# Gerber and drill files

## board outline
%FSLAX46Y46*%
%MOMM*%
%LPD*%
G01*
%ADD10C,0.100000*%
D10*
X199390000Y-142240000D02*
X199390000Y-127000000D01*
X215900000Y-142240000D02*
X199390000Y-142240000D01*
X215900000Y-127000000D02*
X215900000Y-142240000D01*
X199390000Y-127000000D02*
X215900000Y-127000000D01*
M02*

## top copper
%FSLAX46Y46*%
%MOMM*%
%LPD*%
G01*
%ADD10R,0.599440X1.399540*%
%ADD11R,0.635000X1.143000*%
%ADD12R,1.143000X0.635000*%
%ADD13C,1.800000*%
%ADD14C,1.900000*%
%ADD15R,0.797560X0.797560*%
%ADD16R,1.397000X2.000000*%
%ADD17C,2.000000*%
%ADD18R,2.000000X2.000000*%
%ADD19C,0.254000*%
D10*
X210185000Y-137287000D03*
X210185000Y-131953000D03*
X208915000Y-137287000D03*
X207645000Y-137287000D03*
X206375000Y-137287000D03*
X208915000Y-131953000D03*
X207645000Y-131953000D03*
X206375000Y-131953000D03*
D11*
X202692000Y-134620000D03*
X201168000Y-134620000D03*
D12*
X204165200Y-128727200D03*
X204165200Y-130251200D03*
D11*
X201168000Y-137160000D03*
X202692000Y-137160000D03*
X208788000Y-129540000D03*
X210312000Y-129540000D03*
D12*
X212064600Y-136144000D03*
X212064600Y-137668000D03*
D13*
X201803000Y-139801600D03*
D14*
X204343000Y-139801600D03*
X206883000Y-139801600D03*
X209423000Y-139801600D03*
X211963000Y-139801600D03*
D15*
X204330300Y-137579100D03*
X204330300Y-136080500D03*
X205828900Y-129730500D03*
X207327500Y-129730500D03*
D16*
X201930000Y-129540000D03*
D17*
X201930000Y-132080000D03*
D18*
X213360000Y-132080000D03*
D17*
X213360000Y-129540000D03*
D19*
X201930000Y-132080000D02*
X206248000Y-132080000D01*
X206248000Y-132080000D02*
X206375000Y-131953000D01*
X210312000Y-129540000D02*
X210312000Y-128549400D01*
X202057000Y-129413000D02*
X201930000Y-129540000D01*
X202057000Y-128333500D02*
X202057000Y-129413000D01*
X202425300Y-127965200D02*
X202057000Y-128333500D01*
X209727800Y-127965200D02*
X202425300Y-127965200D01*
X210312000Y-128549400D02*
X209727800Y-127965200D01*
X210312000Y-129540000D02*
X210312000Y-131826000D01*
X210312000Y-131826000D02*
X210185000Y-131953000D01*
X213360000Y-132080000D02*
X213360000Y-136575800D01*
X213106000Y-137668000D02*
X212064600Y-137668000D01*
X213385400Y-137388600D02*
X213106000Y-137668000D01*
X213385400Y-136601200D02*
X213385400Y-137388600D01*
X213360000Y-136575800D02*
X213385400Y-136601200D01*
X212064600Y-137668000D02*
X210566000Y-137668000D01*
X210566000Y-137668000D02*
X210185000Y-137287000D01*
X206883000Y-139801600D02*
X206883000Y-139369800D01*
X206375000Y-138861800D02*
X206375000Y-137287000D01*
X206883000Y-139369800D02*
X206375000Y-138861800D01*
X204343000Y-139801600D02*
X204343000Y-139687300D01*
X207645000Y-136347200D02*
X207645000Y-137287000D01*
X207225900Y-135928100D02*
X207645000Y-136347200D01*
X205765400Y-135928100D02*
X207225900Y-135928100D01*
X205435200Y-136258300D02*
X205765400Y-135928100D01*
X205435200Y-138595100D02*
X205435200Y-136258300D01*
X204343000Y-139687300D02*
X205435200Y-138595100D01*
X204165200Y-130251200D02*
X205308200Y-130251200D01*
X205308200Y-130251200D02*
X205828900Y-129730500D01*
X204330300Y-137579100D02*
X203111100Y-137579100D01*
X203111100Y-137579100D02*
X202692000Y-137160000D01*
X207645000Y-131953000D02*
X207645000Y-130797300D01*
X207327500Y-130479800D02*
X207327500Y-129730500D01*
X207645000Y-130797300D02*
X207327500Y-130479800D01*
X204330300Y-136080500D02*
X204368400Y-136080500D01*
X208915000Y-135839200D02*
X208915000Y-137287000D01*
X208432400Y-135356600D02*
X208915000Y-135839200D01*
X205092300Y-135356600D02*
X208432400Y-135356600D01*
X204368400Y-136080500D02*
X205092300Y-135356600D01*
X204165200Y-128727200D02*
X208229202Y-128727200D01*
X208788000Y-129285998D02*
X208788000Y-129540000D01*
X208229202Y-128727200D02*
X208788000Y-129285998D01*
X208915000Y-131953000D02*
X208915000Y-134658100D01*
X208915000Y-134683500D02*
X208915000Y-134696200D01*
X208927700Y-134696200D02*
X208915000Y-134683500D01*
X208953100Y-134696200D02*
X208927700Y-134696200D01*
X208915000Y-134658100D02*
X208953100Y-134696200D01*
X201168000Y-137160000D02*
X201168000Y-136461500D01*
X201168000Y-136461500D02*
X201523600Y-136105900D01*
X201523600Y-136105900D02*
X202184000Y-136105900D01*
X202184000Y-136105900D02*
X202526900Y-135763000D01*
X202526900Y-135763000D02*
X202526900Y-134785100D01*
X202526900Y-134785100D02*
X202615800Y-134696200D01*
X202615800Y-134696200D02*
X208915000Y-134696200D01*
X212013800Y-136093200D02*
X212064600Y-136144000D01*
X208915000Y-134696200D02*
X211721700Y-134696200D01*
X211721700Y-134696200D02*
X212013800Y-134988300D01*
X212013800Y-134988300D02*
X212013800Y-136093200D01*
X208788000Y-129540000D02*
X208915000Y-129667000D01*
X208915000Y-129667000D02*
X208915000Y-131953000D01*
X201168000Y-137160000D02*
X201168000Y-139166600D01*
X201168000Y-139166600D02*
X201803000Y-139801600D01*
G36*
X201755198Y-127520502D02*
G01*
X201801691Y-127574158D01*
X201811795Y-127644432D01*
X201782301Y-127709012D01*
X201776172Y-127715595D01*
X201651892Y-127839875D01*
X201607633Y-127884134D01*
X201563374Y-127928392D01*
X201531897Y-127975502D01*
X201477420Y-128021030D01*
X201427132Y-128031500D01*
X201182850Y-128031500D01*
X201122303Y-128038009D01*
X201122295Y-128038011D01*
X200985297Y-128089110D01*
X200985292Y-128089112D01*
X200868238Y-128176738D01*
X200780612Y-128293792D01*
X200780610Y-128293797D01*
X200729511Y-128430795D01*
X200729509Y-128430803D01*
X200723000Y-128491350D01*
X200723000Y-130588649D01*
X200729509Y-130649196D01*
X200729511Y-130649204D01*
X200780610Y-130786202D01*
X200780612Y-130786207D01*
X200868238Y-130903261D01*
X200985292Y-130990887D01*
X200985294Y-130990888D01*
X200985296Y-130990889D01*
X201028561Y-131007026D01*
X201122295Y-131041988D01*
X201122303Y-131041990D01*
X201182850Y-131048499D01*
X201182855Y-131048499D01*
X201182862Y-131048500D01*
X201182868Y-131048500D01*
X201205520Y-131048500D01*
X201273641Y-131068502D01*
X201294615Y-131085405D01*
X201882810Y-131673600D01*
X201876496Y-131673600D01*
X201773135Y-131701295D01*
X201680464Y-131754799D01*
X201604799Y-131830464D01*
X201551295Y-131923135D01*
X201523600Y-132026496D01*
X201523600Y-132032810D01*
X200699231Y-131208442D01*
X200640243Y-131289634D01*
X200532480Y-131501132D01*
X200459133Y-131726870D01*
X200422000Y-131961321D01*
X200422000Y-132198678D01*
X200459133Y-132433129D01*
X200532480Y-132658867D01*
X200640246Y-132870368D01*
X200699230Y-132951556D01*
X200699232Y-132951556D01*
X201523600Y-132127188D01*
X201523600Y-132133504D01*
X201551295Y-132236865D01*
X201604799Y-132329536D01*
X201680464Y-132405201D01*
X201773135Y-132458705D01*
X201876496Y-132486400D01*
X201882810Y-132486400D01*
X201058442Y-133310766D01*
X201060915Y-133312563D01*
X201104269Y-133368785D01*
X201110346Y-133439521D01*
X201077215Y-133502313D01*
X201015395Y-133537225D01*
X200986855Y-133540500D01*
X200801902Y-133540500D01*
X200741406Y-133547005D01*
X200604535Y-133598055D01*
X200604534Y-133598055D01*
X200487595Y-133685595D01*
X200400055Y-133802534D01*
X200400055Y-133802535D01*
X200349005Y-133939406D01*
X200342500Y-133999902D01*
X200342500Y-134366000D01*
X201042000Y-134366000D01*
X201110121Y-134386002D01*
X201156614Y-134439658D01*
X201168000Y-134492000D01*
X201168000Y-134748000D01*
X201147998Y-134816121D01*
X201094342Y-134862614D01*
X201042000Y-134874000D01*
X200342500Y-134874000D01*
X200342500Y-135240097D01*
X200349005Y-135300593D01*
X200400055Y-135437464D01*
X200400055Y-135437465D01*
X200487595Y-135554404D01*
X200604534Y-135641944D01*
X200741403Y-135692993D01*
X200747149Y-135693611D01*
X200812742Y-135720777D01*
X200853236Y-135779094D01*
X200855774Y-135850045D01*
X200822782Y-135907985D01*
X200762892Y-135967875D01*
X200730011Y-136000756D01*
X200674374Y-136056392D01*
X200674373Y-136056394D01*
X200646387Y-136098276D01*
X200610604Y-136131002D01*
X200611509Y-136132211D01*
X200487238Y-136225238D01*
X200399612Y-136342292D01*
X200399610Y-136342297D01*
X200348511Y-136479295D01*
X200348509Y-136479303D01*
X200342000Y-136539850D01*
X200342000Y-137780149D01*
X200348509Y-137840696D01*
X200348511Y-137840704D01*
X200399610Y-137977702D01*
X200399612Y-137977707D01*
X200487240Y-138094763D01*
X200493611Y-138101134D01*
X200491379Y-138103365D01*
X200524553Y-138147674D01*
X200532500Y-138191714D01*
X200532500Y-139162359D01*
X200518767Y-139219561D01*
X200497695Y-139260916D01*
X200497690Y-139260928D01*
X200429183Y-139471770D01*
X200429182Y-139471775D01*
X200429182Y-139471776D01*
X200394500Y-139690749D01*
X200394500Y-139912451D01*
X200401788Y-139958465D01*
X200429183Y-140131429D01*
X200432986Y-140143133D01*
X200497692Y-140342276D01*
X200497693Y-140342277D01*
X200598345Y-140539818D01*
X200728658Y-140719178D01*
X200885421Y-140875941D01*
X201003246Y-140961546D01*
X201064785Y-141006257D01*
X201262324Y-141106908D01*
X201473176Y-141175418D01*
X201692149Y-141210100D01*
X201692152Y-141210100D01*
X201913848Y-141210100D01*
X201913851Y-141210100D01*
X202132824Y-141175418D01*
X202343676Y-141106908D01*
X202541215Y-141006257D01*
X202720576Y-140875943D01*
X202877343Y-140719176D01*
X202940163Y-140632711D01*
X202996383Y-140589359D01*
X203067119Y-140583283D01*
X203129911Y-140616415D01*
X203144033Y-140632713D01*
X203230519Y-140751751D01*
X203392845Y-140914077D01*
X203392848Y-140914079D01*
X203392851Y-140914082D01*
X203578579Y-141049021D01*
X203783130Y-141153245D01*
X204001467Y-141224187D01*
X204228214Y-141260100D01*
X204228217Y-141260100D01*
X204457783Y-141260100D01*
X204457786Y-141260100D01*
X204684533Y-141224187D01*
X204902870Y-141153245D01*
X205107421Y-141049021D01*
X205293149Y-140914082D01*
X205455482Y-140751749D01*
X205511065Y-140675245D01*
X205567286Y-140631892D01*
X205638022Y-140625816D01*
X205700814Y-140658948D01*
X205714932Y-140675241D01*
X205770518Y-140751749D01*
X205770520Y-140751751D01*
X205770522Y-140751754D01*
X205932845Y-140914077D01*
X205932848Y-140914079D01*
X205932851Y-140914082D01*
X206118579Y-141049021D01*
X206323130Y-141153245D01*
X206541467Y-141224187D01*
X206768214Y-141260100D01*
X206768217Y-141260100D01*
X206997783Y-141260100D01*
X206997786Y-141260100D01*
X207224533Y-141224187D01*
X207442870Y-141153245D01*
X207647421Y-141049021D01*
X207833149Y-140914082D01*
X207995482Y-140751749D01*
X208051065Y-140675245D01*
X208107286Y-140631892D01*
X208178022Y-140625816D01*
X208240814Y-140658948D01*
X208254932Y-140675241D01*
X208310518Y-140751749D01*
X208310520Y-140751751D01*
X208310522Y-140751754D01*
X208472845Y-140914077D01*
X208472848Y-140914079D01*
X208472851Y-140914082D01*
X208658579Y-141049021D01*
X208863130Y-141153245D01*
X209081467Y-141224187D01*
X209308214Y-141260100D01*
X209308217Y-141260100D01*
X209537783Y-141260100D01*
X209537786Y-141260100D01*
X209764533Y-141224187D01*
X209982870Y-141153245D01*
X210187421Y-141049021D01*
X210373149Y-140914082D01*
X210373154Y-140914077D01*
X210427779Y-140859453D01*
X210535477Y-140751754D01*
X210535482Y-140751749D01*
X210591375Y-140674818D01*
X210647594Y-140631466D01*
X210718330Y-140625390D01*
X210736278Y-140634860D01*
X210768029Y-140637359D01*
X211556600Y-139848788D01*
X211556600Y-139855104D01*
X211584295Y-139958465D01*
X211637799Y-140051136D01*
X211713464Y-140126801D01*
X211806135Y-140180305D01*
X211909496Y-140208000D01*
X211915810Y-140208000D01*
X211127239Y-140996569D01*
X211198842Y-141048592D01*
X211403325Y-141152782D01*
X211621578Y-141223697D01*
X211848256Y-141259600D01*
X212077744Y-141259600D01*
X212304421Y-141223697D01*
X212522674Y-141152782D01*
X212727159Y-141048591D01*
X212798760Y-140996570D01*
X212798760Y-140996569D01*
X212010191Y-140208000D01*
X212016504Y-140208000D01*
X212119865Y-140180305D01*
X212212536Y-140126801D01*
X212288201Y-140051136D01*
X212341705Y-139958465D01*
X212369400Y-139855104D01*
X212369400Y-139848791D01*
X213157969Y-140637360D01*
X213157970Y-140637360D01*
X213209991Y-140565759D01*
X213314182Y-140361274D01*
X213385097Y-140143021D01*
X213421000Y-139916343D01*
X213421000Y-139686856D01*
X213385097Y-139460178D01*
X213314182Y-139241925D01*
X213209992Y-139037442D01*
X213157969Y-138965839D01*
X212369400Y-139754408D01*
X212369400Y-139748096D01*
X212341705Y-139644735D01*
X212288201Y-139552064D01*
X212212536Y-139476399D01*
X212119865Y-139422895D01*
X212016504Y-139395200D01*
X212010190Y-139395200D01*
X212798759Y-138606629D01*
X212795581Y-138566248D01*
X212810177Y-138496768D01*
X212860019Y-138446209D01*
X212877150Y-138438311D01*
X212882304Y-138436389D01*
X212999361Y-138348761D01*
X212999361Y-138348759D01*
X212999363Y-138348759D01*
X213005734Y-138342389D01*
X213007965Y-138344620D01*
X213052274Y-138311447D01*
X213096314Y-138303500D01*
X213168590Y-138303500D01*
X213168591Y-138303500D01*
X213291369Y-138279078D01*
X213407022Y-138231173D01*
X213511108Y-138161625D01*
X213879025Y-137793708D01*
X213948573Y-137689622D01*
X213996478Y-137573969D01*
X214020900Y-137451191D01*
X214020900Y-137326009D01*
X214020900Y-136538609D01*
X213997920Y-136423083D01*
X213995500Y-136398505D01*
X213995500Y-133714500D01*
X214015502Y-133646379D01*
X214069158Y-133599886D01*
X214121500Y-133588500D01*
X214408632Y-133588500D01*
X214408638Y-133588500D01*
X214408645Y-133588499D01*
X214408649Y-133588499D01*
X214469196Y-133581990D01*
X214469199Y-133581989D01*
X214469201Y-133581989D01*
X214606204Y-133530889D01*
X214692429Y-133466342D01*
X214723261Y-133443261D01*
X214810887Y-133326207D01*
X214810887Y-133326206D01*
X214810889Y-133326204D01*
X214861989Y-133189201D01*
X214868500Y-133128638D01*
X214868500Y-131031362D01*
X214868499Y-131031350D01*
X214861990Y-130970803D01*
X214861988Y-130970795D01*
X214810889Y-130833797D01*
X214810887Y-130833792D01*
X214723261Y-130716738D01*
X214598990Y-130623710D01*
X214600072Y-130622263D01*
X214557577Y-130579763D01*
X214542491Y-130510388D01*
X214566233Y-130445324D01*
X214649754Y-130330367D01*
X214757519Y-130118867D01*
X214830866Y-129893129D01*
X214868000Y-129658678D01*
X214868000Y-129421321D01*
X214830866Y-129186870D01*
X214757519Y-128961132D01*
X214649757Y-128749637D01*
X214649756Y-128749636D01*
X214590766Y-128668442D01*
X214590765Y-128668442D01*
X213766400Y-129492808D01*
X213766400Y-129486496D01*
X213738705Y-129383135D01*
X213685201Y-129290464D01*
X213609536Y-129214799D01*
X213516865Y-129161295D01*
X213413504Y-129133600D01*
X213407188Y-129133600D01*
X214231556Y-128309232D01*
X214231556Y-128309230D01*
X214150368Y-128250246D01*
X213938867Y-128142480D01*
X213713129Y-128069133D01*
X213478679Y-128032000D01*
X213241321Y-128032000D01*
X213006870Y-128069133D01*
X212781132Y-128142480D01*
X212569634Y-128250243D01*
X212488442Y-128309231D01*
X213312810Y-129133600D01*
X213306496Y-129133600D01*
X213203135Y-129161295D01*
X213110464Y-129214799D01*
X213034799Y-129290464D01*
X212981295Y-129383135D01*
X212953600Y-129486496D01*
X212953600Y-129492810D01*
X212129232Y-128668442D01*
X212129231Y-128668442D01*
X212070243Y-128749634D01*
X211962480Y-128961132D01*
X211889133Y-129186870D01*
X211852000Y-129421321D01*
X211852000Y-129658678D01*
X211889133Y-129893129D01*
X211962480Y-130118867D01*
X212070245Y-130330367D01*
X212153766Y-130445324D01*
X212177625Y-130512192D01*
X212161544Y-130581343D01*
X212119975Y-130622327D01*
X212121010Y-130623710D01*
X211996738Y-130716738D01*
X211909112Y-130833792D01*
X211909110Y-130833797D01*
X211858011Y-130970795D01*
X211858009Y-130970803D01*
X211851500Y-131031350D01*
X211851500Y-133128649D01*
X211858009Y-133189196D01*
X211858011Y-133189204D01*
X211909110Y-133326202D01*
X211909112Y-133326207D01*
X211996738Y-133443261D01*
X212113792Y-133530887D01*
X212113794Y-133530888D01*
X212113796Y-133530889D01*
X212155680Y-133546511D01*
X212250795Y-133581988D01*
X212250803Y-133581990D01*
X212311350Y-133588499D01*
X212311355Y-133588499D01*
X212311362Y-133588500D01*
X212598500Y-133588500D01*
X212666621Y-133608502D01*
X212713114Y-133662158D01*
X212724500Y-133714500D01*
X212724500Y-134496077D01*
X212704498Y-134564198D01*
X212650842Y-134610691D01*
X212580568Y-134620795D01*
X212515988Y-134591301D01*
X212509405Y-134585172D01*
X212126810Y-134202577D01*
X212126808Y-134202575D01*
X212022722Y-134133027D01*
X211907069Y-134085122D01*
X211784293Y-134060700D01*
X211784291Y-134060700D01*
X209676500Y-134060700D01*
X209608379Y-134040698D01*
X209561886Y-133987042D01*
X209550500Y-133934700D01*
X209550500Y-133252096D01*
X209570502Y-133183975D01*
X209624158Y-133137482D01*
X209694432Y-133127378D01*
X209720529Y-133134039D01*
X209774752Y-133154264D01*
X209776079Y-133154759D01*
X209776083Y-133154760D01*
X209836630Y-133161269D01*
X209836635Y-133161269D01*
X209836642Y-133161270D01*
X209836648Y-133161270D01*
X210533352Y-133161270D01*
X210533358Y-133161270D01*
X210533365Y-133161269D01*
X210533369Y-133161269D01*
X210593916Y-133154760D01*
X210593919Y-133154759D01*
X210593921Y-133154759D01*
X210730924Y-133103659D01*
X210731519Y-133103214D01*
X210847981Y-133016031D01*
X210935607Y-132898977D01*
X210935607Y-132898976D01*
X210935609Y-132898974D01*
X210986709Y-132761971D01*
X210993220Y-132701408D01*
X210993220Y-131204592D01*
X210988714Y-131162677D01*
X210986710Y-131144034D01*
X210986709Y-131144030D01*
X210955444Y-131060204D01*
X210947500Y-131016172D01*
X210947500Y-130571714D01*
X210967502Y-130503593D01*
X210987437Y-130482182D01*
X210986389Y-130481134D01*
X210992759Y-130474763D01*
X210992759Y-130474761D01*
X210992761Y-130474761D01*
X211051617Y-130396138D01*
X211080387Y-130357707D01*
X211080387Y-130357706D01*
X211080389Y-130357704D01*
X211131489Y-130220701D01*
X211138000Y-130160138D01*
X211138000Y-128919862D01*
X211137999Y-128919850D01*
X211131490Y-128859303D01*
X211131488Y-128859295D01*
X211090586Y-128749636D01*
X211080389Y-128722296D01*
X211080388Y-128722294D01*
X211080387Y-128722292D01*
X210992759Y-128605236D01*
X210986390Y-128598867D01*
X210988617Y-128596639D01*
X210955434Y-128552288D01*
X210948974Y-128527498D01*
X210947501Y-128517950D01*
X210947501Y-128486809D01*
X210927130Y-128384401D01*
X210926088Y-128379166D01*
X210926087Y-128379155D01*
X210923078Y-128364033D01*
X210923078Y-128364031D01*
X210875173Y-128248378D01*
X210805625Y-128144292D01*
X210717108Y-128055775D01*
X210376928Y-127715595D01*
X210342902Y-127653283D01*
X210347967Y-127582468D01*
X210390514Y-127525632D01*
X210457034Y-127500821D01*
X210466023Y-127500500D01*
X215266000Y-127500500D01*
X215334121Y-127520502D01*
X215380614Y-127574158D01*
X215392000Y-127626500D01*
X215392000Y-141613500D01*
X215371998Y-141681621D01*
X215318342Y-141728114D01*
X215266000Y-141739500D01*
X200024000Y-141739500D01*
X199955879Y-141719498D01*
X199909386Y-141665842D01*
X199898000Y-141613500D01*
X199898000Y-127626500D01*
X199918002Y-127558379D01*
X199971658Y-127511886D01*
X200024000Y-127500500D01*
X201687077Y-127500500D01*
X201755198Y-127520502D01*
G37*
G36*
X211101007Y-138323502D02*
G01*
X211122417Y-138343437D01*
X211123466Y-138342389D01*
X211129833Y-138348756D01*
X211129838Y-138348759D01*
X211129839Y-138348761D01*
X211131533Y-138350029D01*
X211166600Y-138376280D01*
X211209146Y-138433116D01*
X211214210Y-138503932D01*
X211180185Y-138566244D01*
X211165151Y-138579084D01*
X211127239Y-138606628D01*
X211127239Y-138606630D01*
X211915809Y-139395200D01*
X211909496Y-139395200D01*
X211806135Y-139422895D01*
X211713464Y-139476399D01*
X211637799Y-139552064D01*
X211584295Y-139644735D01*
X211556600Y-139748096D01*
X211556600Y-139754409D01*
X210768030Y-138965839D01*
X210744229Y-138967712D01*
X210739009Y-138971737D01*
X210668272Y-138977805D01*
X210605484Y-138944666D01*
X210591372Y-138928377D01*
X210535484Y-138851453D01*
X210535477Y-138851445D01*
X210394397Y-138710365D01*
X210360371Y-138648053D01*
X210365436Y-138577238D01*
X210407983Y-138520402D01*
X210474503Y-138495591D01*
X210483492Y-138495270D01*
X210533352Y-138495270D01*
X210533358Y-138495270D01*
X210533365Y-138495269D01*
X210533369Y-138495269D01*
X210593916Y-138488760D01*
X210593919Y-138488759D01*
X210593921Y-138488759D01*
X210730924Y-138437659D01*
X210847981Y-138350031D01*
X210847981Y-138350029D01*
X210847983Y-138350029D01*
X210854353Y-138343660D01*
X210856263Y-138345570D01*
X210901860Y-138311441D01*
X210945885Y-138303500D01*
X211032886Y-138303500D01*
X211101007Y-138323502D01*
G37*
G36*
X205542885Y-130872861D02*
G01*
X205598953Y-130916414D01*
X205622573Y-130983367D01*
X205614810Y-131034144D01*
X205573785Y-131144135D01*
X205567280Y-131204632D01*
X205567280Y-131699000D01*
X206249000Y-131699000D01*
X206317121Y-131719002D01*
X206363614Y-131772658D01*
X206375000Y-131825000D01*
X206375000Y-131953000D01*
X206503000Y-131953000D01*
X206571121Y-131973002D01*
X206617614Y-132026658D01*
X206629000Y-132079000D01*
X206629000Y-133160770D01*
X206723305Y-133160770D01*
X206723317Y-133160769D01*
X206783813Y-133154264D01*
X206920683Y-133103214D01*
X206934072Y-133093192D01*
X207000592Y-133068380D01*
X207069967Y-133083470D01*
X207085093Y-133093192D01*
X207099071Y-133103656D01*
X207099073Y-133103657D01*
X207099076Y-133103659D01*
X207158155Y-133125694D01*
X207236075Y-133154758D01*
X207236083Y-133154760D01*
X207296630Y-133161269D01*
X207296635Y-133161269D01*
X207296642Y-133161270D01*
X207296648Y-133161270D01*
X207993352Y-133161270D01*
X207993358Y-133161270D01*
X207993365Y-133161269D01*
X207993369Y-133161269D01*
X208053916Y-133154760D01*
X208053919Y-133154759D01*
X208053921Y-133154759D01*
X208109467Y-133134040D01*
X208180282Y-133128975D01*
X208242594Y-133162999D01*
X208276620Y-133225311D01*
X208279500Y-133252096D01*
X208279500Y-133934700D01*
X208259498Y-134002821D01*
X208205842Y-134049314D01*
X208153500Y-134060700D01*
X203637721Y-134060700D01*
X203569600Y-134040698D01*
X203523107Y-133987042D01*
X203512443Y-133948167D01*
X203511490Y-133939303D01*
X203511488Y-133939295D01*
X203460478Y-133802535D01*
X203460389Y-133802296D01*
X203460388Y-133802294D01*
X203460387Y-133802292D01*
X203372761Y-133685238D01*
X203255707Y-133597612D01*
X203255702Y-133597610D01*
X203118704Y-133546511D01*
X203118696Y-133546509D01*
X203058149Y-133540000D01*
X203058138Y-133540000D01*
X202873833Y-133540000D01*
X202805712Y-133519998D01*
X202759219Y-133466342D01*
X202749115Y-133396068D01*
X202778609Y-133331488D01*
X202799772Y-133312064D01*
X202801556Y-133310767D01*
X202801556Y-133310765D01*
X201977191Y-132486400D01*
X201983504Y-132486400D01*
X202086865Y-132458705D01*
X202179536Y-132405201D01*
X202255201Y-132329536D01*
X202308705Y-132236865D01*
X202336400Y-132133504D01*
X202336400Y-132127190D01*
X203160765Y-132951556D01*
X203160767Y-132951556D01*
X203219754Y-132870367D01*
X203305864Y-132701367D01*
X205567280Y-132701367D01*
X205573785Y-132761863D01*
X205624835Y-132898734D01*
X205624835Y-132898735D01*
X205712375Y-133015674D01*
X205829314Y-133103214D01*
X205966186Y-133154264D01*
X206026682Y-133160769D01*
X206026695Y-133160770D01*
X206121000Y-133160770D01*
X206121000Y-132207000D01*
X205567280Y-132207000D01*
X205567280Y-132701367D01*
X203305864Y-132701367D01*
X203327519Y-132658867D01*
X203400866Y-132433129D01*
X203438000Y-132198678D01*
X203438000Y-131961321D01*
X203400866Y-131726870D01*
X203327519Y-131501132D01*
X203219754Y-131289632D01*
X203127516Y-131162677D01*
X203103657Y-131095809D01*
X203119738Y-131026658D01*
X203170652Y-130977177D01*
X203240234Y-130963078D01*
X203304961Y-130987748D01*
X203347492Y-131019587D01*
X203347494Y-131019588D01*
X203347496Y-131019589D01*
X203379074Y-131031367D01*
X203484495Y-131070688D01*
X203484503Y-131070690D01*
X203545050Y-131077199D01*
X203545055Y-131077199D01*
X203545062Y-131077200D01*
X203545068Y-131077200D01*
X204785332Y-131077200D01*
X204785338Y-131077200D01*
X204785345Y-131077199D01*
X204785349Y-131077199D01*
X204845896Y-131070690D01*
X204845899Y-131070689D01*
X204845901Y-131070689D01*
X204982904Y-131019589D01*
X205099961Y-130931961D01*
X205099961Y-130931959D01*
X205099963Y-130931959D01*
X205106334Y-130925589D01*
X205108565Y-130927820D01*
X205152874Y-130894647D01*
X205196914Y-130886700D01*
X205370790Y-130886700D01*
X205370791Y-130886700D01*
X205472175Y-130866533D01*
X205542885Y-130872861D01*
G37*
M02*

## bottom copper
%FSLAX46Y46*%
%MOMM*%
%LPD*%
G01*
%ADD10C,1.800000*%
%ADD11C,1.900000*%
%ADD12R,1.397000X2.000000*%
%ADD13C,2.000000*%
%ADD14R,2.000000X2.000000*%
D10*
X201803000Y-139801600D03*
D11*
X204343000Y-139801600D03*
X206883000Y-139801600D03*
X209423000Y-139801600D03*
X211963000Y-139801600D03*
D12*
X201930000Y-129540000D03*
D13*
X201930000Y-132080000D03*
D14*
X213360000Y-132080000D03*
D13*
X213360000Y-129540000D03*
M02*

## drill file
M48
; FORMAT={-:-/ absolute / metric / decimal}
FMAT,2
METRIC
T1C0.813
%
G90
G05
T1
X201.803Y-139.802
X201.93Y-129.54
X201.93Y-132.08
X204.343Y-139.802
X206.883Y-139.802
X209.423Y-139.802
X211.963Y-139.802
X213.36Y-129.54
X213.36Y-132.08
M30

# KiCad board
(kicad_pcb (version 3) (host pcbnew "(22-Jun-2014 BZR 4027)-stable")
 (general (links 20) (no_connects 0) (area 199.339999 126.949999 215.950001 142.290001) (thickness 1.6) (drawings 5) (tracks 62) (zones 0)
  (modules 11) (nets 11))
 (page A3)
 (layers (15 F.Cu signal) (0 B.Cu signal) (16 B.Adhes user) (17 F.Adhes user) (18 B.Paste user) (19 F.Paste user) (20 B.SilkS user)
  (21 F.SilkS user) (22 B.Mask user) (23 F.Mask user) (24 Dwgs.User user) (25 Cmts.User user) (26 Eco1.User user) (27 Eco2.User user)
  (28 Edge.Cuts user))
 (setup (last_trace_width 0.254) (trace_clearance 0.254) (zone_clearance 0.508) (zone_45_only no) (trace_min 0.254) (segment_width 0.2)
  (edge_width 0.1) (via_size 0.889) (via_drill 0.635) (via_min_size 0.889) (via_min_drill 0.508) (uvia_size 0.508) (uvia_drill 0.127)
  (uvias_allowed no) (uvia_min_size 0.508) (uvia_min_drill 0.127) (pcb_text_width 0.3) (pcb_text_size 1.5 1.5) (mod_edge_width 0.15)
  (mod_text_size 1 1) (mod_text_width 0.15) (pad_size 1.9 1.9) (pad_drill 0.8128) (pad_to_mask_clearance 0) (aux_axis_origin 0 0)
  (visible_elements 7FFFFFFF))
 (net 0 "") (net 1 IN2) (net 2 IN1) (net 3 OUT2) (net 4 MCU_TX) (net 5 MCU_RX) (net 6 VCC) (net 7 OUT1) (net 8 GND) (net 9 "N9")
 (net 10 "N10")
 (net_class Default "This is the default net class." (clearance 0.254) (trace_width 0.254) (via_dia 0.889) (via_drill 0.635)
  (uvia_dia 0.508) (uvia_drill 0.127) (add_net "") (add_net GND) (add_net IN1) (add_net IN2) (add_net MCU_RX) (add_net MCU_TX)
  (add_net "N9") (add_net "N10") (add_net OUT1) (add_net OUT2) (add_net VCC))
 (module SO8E (layer F.Cu) (at 208.28 134.62 180)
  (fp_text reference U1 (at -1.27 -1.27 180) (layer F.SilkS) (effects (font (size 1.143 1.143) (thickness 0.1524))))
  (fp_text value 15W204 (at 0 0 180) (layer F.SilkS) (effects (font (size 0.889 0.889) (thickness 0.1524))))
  (pad 8 smd rect (at -1.905 -2.667 180) (size 0.59944 1.39954) (layers F.Cu F.Paste F.Mask) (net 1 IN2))
  (pad 1 smd rect (at -1.905 2.667 180) (size 0.59944 1.39954) (layers F.Cu F.Paste F.Mask) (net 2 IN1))
  (pad 7 smd rect (at -0.635 -2.667 180) (size 0.59944 1.39954) (layers F.Cu F.Paste F.Mask) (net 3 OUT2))
  (pad 6 smd rect (at 0.635 -2.667 180) (size 0.59944 1.39954) (layers F.Cu F.Paste F.Mask) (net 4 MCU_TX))
  (pad 5 smd rect (at 1.905 -2.667 180) (size 0.59944 1.39954) (layers F.Cu F.Paste F.Mask) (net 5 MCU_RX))
  (pad 2 smd rect (at -0.635 2.667 180) (size 0.59944 1.39954) (layers F.Cu F.Paste F.Mask) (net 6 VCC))
  (pad 3 smd rect (at 0.635 2.667 180) (size 0.59944 1.39954) (layers F.Cu F.Paste F.Mask) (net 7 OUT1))
  (pad 4 smd rect (at 1.905 2.667 180) (size 0.59944 1.39954) (layers F.Cu F.Paste F.Mask) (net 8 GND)))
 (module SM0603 (layer F.Cu) (at 201.93 134.62 180)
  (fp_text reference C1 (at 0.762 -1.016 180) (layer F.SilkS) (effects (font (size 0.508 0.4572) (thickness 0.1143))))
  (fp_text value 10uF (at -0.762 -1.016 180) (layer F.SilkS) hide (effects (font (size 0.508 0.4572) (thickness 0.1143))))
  (pad 1 smd rect (at -0.762 0 180) (size 0.635 1.143) (layers F.Cu F.Paste F.Mask) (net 6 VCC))
  (pad 2 smd rect (at 0.762 0 180) (size 0.635 1.143) (layers F.Cu F.Paste F.Mask) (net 8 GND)))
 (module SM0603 (layer F.Cu) (at 204.1652 129.4892 270)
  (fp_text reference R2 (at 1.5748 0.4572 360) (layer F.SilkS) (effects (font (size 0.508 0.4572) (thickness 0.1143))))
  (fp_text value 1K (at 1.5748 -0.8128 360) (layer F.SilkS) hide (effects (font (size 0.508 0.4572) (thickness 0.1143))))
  (pad 1 smd rect (at -0.762 0 270) (size 0.635 1.143) (layers F.Cu F.Paste F.Mask) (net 6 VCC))
  (pad 2 smd rect (at 0.762 0 270) (size 0.635 1.143) (layers F.Cu F.Paste F.Mask) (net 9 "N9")))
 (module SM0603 (layer F.Cu) (at 201.93 137.16)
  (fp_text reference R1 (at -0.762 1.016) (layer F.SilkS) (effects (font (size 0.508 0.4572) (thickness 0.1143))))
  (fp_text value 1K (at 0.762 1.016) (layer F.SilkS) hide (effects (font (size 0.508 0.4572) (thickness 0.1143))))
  (pad 1 smd rect (at -0.762 0) (size 0.635 1.143) (layers F.Cu F.Paste F.Mask) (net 6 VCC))
  (pad 2 smd rect (at 0.762 0) (size 0.635 1.143) (layers F.Cu F.Paste F.Mask) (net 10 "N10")))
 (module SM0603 (layer F.Cu) (at 209.55 129.54)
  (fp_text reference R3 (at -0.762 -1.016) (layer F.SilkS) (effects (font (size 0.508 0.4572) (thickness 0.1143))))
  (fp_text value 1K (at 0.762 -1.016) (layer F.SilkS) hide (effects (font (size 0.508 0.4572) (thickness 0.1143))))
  (pad 1 smd rect (at -0.762 0) (size 0.635 1.143) (layers F.Cu F.Paste F.Mask) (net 6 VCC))
  (pad 2 smd rect (at 0.762 0) (size 0.635 1.143) (layers F.Cu F.Paste F.Mask) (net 2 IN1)))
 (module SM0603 (layer F.Cu) (at 212.0646 136.906 270)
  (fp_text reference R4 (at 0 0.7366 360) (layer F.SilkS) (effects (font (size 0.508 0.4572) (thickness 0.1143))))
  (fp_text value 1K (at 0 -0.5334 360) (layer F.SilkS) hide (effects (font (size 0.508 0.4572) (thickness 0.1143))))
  (pad 1 smd rect (at -0.762 0 270) (size 0.635 1.143) (layers F.Cu F.Paste F.Mask) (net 6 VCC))
  (pad 2 smd rect (at 0.762 0 270) (size 0.635 1.143) (layers F.Cu F.Paste F.Mask) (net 1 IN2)))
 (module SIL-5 (layer F.Cu) (at 208.153 139.8016)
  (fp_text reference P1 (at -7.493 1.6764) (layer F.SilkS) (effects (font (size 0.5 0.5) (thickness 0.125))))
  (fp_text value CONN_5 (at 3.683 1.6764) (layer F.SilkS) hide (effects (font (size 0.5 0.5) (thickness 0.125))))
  (pad 1 thru_hole circle (at -6.35 0) (size 1.8 1.8) (drill 0.8128) (layers *.Mask F.Cu F.SilkS) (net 6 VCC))
  (pad 2 thru_hole circle (at -3.81 0) (size 1.9 1.9) (drill 0.8128) (layers *.Mask F.Cu F.SilkS) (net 4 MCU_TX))
  (pad 3 thru_hole circle (at -1.27 0) (size 1.9 1.9) (drill 0.8128) (layers *.Mask F.Cu F.Adhes F.Paste F.SilkS) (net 5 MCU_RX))
  (pad 4 thru_hole circle (at 1.27 0) (size 1.9 1.9) (drill 0.8128) (layers *.Mask F.Cu F.SilkS))
  (pad 5 thru_hole circle (at 3.81 0) (size 1.9 1.9) (drill 0.8128) (layers *.Mask F.Cu F.SilkS) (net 8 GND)))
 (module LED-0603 (layer F.Cu) (at 204.3303 136.8298 90)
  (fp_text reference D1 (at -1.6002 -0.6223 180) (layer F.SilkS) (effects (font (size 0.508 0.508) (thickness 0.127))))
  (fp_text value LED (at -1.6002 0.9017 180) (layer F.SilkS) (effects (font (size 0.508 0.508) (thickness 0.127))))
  (pad 1 smd rect (at -0.7493 0 90) (size 0.79756 0.79756) (layers F.Cu F.Paste F.Mask) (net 10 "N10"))
  (pad 2 smd rect (at 0.7493 0 90) (size 0.79756 0.79756) (layers F.Cu F.Paste F.Mask) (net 3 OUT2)))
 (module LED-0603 (layer F.Cu) (at 206.5782 129.7305)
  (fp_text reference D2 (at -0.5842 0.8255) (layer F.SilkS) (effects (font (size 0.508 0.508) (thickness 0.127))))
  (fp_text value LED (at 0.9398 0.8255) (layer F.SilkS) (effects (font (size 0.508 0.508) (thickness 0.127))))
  (pad 1 smd rect (at -0.7493 0) (size 0.79756 0.79756) (layers F.Cu F.Paste F.Mask) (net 9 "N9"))
  (pad 2 smd rect (at 0.7493 0) (size 0.79756 0.79756) (layers F.Cu F.Paste F.Mask) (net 7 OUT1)))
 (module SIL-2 (layer F.Cu) (at 201.93 130.81 270)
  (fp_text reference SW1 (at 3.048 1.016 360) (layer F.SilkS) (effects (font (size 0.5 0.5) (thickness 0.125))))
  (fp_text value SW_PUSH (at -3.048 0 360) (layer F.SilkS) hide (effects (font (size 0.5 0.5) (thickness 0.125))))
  (pad 1 thru_hole rect (at -1.27 0 270) (size 2 1.397) (drill 0.8128) (layers *.Mask F.Cu F.SilkS) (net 2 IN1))
  (pad 2 thru_hole circle (at 1.27 0 270) (size 2 2) (drill 0.8128) (layers *.Mask F.Cu F.SilkS) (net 8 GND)))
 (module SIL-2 (layer F.Cu) (at 213.36 130.81 90)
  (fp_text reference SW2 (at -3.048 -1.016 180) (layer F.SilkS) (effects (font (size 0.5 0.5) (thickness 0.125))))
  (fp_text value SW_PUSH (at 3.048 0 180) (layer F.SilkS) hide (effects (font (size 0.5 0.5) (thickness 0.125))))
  (pad 1 thru_hole rect (at -1.27 0 90) (size 2 2) (drill 0.8128) (layers *.Mask F.Cu F.SilkS) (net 1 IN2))
  (pad 2 thru_hole circle (at 1.27 0 90) (size 2 2) (drill 0.8128) (layers *.Mask F.Cu F.SilkS) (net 8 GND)))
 (gr_line (start 199.39 142.24) (end 199.39 127) (angle 90) (layer Edge.Cuts) (width 0.1))
 (gr_line (start 215.9 142.24) (end 199.39 142.24) (angle 90) (layer Edge.Cuts) (width 0.1))
 (gr_line (start 215.9 127) (end 215.9 142.24) (angle 90) (layer Edge.Cuts) (width 0.1))
 (gr_line (start 199.39 127) (end 215.9 127) (angle 90) (layer Edge.Cuts) (width 0.1))
 (segment (start 201.93 132.08) (end 206.248 132.08) (width 0.254) (layer F.Cu) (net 8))
 (segment (start 206.248 132.08) (end 206.375 131.953) (width 0.254) (layer F.Cu) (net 8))
 (segment (start 210.312 129.54) (end 210.312 128.5494) (width 0.254) (layer F.Cu) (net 2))
 (segment (start 202.057 129.413) (end 201.93 129.54) (width 0.254) (layer F.Cu) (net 2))
 (segment (start 202.057 128.3335) (end 202.057 129.413) (width 0.254) (layer F.Cu) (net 2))
 (segment (start 202.4253 127.9652) (end 202.057 128.3335) (width 0.254) (layer F.Cu) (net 2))
 (segment (start 209.7278 127.9652) (end 202.4253 127.9652) (width 0.254) (layer F.Cu) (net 2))
 (segment (start 210.312 128.5494) (end 209.7278 127.9652) (width 0.254) (layer F.Cu) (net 2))
 (segment (start 210.312 129.54) (end 210.312 131.826) (width 0.254) (layer F.Cu) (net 2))
 (segment (start 210.312 131.826) (end 210.185 131.953) (width 0.254) (layer F.Cu) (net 2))
 (segment (start 213.36 132.08) (end 213.36 136.5758) (width 0.254) (layer F.Cu) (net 1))
 (segment (start 213.106 137.668) (end 212.0646 137.668) (width 0.254) (layer F.Cu) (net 1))
 (segment (start 213.3854 137.3886) (end 213.106 137.668) (width 0.254) (layer F.Cu) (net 1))
 (segment (start 213.3854 136.6012) (end 213.3854 137.3886) (width 0.254) (layer F.Cu) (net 1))
 (segment (start 213.36 136.5758) (end 213.3854 136.6012) (width 0.254) (layer F.Cu) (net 1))
 (segment (start 212.0646 137.668) (end 210.566 137.668) (width 0.254) (layer F.Cu) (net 1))
 (segment (start 210.566 137.668) (end 210.185 137.287) (width 0.254) (layer F.Cu) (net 1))
 (segment (start 206.883 139.8016) (end 206.883 139.3698) (width 0.254) (layer F.Cu) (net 5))
 (segment (start 206.375 138.8618) (end 206.375 137.287) (width 0.254) (layer F.Cu) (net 5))
 (segment (start 206.883 139.3698) (end 206.375 138.8618) (width 0.254) (layer F.Cu) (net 5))
 (segment (start 204.343 139.8016) (end 204.343 139.6873) (width 0.254) (layer F.Cu) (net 4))
 (segment (start 207.645 136.3472) (end 207.645 137.287) (width 0.254) (layer F.Cu) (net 4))
 (segment (start 207.2259 135.9281) (end 207.645 136.3472) (width 0.254) (layer F.Cu) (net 4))
 (segment (start 205.7654 135.9281) (end 207.2259 135.9281) (width 0.254) (layer F.Cu) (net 4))
 (segment (start 205.4352 136.2583) (end 205.7654 135.9281) (width 0.254) (layer F.Cu) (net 4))
 (segment (start 205.4352 138.5951) (end 205.4352 136.2583) (width 0.254) (layer F.Cu) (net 4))
 (segment (start 204.343 139.6873) (end 205.4352 138.5951) (width 0.254) (layer F.Cu) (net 4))
 (segment (start 204.1652 130.2512) (end 205.3082 130.2512) (width 0.254) (layer F.Cu) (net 9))
 (segment (start 205.3082 130.2512) (end 205.8289 129.7305) (width 0.254) (layer F.Cu) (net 9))
 (segment (start 204.3303 137.5791) (end 203.1111 137.5791) (width 0.254) (layer F.Cu) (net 10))
 (segment (start 203.1111 137.5791) (end 202.692 137.16) (width 0.254) (layer F.Cu) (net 10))
 (segment (start 207.645 131.953) (end 207.645 130.7973) (width 0.254) (layer F.Cu) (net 7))
 (segment (start 207.3275 130.4798) (end 207.3275 129.7305) (width 0.254) (layer F.Cu) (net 7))
 (segment (start 207.645 130.7973) (end 207.3275 130.4798) (width 0.254) (layer F.Cu) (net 7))
 (segment (start 204.3303 136.0805) (end 204.3684 136.0805) (width 0.254) (layer F.Cu) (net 3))
 (segment (start 208.915 135.8392) (end 208.915 137.287) (width 0.254) (layer F.Cu) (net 3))
 (segment (start 208.4324 135.3566) (end 208.915 135.8392) (width 0.254) (layer F.Cu) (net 3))
 (segment (start 205.0923 135.3566) (end 208.4324 135.3566) (width 0.254) (layer F.Cu) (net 3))
 (segment (start 204.3684 136.0805) (end 205.0923 135.3566) (width 0.254) (layer F.Cu) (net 3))
 (segment (start 204.1652 128.7272) (end 208.229202 128.7272) (width 0.254) (layer F.Cu) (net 6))
 (segment (start 208.788 129.285998) (end 208.788 129.54) (width 0.254) (layer F.Cu) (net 6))
 (segment (start 208.229202 128.7272) (end 208.788 129.285998) (width 0.254) (layer F.Cu) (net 6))
 (segment (start 208.915 131.953) (end 208.915 134.6581) (width 0.254) (layer F.Cu) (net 6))
 (segment (start 208.915 134.6835) (end 208.915 134.6962) (width 0.254) (layer F.Cu) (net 6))
 (segment (start 208.9277 134.6962) (end 208.915 134.6835) (width 0.254) (layer F.Cu) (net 6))
 (segment (start 208.9531 134.6962) (end 208.9277 134.6962) (width 0.254) (layer F.Cu) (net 6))
 (segment (start 208.915 134.6581) (end 208.9531 134.6962) (width 0.254) (layer F.Cu) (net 6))
 (segment (start 201.168 137.16) (end 201.168 136.4615) (width 0.254) (layer F.Cu) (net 6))
 (segment (start 201.168 136.4615) (end 201.5236 136.1059) (width 0.254) (layer F.Cu) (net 6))
 (segment (start 201.5236 136.1059) (end 202.184 136.1059) (width 0.254) (layer F.Cu) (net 6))
 (segment (start 202.184 136.1059) (end 202.5269 135.763) (width 0.254) (layer F.Cu) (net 6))
 (segment (start 202.5269 135.763) (end 202.5269 134.7851) (width 0.254) (layer F.Cu) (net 6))
 (segment (start 202.5269 134.7851) (end 202.6158 134.6962) (width 0.254) (layer F.Cu) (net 6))
 (segment (start 202.6158 134.6962) (end 208.915 134.6962) (width 0.254) (layer F.Cu) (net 6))
 (segment (start 212.0138 136.0932) (end 212.0646 136.144) (width 0.254) (layer F.Cu) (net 6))
 (segment (start 208.915 134.6962) (end 211.7217 134.6962) (width 0.254) (layer F.Cu) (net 6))
 (segment (start 211.7217 134.6962) (end 212.0138 134.9883) (width 0.254) (layer F.Cu) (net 6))
 (segment (start 212.0138 134.9883) (end 212.0138 136.0932) (width 0.254) (layer F.Cu) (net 6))
 (segment (start 208.788 129.54) (end 208.915 129.667) (width 0.254) (layer F.Cu) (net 6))
 (segment (start 208.915 129.667) (end 208.915 131.953) (width 0.254) (layer F.Cu) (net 6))
 (segment (start 201.168 137.16) (end 201.168 139.1666) (width 0.254) (layer F.Cu) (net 6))
 (segment (start 201.168 139.1666) (end 201.803 139.8016) (width 0.254) (layer F.Cu) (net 6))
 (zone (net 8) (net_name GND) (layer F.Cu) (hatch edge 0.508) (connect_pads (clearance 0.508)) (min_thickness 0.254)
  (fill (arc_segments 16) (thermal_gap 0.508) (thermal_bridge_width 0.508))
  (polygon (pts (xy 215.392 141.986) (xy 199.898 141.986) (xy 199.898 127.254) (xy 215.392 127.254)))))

